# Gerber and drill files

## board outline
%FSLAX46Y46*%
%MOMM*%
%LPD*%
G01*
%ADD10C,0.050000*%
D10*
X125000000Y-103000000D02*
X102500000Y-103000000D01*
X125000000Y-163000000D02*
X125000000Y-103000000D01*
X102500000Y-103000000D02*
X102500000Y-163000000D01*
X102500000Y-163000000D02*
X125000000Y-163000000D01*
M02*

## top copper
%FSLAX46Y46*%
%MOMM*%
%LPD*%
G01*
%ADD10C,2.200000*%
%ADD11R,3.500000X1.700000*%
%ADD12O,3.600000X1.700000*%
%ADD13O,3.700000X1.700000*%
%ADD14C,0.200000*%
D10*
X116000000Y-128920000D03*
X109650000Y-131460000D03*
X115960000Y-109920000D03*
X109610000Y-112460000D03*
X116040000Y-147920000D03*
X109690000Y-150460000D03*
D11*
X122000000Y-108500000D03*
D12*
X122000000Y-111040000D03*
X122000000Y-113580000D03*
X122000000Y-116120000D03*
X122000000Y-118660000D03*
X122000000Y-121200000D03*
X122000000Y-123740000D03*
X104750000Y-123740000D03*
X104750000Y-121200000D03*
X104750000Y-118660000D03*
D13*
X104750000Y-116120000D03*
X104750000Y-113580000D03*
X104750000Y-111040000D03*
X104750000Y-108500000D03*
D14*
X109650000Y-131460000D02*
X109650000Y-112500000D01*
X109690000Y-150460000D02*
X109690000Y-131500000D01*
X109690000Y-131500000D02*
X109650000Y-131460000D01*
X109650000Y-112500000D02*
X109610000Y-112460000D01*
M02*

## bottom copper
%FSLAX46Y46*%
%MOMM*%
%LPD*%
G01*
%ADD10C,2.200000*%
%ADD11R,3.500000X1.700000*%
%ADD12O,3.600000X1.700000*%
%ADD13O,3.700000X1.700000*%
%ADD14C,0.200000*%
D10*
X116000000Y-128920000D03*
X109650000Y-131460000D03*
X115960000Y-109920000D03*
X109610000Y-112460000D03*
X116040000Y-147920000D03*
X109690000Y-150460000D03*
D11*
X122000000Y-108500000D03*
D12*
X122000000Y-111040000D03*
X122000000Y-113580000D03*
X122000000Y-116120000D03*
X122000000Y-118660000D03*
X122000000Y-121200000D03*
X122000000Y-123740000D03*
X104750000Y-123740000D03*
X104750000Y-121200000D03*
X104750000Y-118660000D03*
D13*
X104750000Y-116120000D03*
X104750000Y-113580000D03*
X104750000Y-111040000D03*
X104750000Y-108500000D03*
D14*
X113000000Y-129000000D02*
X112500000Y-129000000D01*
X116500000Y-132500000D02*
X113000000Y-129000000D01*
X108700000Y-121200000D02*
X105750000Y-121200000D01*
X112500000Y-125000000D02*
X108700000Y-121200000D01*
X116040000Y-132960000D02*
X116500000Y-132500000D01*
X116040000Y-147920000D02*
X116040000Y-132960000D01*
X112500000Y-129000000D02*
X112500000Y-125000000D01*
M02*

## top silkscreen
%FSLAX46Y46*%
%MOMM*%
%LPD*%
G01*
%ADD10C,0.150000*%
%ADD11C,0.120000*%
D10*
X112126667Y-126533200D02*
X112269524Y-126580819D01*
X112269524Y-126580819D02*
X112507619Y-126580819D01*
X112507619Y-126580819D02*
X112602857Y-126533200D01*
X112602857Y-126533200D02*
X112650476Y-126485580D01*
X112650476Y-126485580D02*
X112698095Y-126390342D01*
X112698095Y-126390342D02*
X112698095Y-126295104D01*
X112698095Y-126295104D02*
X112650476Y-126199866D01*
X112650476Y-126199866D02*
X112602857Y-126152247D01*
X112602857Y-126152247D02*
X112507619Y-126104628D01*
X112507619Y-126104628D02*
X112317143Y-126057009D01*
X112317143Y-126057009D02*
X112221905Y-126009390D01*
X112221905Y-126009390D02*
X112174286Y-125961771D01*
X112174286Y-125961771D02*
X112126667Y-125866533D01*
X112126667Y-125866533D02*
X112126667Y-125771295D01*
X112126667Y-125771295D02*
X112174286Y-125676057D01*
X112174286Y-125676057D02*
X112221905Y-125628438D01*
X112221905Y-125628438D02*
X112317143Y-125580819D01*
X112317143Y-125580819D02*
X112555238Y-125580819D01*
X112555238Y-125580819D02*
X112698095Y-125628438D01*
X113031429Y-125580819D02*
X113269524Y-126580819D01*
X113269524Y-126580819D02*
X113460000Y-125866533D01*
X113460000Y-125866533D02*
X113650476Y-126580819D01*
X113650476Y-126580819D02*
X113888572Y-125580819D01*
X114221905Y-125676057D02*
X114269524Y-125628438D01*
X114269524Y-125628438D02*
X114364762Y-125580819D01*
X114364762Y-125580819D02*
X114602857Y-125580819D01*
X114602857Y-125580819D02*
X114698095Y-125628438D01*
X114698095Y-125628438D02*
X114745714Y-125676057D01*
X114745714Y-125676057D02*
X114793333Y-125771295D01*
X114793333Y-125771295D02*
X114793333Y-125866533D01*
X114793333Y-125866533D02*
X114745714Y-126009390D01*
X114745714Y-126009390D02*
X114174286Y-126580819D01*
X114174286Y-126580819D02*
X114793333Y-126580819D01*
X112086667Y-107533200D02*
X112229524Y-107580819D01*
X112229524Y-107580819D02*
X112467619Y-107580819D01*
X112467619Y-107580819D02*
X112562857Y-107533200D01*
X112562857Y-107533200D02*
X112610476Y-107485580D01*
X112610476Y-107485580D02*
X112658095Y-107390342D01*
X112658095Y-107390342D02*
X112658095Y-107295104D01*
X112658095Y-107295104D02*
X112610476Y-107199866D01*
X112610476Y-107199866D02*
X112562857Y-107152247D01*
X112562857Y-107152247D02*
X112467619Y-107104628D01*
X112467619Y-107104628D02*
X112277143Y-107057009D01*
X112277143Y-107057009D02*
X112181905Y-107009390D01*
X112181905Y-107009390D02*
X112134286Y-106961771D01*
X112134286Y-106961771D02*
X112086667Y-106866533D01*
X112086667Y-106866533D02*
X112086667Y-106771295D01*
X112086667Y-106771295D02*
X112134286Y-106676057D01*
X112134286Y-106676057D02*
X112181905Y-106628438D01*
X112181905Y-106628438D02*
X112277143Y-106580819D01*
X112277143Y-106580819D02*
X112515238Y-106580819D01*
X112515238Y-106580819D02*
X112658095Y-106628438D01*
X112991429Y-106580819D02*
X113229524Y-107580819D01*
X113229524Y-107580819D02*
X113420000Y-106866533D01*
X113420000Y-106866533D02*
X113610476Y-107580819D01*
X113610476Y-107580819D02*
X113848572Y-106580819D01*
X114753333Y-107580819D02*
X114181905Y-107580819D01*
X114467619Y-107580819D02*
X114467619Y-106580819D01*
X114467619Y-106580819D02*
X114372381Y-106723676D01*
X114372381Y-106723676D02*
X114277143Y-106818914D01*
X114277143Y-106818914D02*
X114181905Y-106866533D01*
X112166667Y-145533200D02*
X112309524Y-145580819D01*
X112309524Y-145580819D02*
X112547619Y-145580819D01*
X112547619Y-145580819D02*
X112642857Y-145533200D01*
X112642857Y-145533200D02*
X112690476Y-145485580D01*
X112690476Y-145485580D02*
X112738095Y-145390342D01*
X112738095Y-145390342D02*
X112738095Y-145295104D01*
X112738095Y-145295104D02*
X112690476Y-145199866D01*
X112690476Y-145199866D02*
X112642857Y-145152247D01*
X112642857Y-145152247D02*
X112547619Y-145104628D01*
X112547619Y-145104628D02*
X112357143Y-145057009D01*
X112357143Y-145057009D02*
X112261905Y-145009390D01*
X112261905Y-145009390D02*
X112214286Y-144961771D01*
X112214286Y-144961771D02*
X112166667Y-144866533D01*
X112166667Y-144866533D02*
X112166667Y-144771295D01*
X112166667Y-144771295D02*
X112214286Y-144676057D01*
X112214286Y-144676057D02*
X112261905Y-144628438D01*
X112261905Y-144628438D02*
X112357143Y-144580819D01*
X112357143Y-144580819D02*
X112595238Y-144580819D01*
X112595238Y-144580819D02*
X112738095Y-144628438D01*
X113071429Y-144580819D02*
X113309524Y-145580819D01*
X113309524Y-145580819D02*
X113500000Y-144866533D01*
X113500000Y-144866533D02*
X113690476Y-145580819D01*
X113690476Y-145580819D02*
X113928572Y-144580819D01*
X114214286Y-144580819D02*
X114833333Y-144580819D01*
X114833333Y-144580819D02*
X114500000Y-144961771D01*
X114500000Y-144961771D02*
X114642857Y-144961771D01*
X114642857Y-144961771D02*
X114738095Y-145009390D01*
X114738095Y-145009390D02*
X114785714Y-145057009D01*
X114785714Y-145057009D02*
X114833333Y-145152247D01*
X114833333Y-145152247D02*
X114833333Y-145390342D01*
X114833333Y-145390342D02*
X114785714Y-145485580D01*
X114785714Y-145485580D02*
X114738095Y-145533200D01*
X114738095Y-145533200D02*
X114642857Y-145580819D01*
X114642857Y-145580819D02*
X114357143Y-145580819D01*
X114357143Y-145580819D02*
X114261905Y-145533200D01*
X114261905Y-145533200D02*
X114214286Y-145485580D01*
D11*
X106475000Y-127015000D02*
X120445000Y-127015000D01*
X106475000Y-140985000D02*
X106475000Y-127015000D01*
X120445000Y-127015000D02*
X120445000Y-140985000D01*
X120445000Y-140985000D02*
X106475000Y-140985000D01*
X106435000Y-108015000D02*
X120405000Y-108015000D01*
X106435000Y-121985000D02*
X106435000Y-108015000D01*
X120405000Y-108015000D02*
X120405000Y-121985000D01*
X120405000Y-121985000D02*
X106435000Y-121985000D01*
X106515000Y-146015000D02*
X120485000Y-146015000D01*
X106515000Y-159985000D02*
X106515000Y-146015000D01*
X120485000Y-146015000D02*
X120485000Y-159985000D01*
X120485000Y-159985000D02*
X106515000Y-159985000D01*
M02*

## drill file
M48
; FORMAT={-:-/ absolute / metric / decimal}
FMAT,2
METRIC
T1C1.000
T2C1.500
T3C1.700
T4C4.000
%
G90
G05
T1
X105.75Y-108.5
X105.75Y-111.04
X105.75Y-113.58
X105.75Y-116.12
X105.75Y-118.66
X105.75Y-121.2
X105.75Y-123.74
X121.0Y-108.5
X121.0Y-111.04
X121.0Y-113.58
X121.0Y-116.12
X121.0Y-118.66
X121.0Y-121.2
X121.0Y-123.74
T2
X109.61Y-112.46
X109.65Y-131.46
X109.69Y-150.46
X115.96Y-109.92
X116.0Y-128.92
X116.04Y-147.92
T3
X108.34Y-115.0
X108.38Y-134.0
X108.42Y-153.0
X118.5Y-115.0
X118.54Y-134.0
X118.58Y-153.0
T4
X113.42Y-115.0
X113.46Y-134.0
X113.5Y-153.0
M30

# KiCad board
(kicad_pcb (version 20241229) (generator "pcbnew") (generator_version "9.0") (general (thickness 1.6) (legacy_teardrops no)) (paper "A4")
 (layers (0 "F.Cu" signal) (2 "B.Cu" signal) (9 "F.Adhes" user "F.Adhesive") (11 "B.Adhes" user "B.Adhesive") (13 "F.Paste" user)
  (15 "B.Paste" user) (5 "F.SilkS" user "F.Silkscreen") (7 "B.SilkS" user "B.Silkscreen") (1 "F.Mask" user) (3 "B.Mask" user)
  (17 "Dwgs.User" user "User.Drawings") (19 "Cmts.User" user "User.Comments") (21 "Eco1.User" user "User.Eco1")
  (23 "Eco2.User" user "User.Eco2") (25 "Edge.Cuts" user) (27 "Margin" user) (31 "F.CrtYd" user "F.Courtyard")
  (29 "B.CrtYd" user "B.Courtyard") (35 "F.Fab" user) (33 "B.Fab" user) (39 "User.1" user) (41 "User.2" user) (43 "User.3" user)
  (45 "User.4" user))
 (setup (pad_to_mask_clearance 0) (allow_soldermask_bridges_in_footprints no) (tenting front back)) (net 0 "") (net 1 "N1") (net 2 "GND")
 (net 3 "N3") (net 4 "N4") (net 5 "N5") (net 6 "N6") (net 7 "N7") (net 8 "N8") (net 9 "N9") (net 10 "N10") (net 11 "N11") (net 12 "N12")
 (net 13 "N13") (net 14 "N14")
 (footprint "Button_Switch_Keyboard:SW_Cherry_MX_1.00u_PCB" (layer "F.Cu") (at 116 128.92)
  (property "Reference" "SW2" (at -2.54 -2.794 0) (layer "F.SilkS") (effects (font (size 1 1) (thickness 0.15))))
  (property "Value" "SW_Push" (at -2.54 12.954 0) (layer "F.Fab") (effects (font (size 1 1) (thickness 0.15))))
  (fp_line (start -9.525 -1.905) (end 4.445 -1.905) (stroke (width 0.12) (type solid)) (layer "F.SilkS"))
  (fp_line (start -9.525 12.065) (end -9.525 -1.905) (stroke (width 0.12) (type solid)) (layer "F.SilkS"))
  (fp_line (start 4.445 -1.905) (end 4.445 12.065) (stroke (width 0.12) (type solid)) (layer "F.SilkS"))
  (fp_line (start 4.445 12.065) (end -9.525 12.065) (stroke (width 0.12) (type solid)) (layer "F.SilkS"))
  (pad "" np_thru_hole circle (at -7.62 5.08) (size 1.7 1.7) (drill 1.7) (layers "*.Cu" "*.Mask"))
  (pad "" np_thru_hole circle (at -2.54 5.08) (size 4 4) (drill 4) (layers "*.Cu" "*.Mask"))
  (pad "" np_thru_hole circle (at 2.54 5.08) (size 1.7 1.7) (drill 1.7) (layers "*.Cu" "*.Mask"))
  (pad "1" thru_hole circle (at 0 0) (size 2.2 2.2) (drill 1.5) (layers "*.Cu" "*.Mask") (remove_unused_layers no) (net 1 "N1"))
  (pad "2" thru_hole circle (at -6.35 2.54) (size 2.2 2.2) (drill 1.5) (layers "*.Cu" "*.Mask") (remove_unused_layers no) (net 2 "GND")))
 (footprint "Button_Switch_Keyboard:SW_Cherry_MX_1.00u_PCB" (layer "F.Cu") (at 115.96 109.92)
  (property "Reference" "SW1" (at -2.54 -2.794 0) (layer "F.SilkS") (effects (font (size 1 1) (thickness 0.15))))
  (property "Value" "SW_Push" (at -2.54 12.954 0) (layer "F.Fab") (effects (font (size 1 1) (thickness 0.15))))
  (fp_line (start -9.525 -1.905) (end 4.445 -1.905) (stroke (width 0.12) (type solid)) (layer "F.SilkS"))
  (fp_line (start -9.525 12.065) (end -9.525 -1.905) (stroke (width 0.12) (type solid)) (layer "F.SilkS"))
  (fp_line (start 4.445 -1.905) (end 4.445 12.065) (stroke (width 0.12) (type solid)) (layer "F.SilkS"))
  (fp_line (start 4.445 12.065) (end -9.525 12.065) (stroke (width 0.12) (type solid)) (layer "F.SilkS"))
  (pad "" np_thru_hole circle (at -7.62 5.08) (size 1.7 1.7) (drill 1.7) (layers "*.Cu" "*.Mask"))
  (pad "" np_thru_hole circle (at -2.54 5.08) (size 4 4) (drill 4) (layers "*.Cu" "*.Mask"))
  (pad "" np_thru_hole circle (at 2.54 5.08) (size 1.7 1.7) (drill 1.7) (layers "*.Cu" "*.Mask"))
  (pad "1" thru_hole circle (at 0 0) (size 2.2 2.2) (drill 1.5) (layers "*.Cu" "*.Mask") (remove_unused_layers no) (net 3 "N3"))
  (pad "2" thru_hole circle (at -6.35 2.54) (size 2.2 2.2) (drill 1.5) (layers "*.Cu" "*.Mask") (remove_unused_layers no) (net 2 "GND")))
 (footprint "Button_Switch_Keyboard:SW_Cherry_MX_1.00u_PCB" (layer "F.Cu") (at 116.04 147.92)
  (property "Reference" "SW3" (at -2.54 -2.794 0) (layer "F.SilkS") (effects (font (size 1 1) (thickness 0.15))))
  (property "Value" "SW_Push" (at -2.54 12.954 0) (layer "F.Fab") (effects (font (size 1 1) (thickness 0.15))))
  (fp_line (start -9.525 -1.905) (end 4.445 -1.905) (stroke (width 0.12) (type solid)) (layer "F.SilkS"))
  (fp_line (start -9.525 12.065) (end -9.525 -1.905) (stroke (width 0.12) (type solid)) (layer "F.SilkS"))
  (fp_line (start 4.445 -1.905) (end 4.445 12.065) (stroke (width 0.12) (type solid)) (layer "F.SilkS"))
  (fp_line (start 4.445 12.065) (end -9.525 12.065) (stroke (width 0.12) (type solid)) (layer "F.SilkS"))
  (pad "" np_thru_hole circle (at -7.62 5.08) (size 1.7 1.7) (drill 1.7) (layers "*.Cu" "*.Mask"))
  (pad "" np_thru_hole circle (at -2.54 5.08) (size 4 4) (drill 4) (layers "*.Cu" "*.Mask"))
  (pad "" np_thru_hole circle (at 2.54 5.08) (size 1.7 1.7) (drill 1.7) (layers "*.Cu" "*.Mask"))
  (pad "1" thru_hole circle (at 0 0) (size 2.2 2.2) (drill 1.5) (layers "*.Cu" "*.Mask") (remove_unused_layers no) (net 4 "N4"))
  (pad "2" thru_hole circle (at -6.35 2.54) (size 2.2 2.2) (drill 1.5) (layers "*.Cu" "*.Mask") (remove_unused_layers no) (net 2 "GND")))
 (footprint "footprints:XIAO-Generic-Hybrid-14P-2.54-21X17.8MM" (layer "B.Cu") (at 113.375 116.12 180)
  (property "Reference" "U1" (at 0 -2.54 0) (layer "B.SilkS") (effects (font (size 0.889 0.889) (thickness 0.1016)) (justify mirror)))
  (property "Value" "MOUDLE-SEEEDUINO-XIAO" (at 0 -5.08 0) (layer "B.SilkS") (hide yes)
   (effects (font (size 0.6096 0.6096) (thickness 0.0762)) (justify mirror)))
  (pad "1" thru_hole rect (at -7.625 7.62 180) (size 3.5 1.7) (drill 1 (offset -1 0)) (layers "*.Cu" "*.Mask") (remove_unused_layers no)
   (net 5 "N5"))
  (pad "2" thru_hole oval (at -7.625 5.08 180) (size 3.6 1.7) (drill 1 (offset -1 0)) (layers "*.Cu" "*.Mask") (remove_unused_layers no)
   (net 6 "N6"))
  (pad "3" thru_hole oval (at -7.625 2.54 180) (size 3.6 1.7) (drill 1 (offset -1 0)) (layers "*.Cu" "*.Mask") (remove_unused_layers no)
   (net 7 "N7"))
  (pad "4" thru_hole oval (at -7.625 0 180) (size 3.6 1.7) (drill 1 (offset -1 0)) (layers "*.Cu" "*.Mask") (remove_unused_layers no)
   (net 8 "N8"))
  (pad "5" thru_hole oval (at -7.625 -2.54 180) (size 3.6 1.7) (drill 1 (offset -1 0)) (layers "*.Cu" "*.Mask") (remove_unused_layers no)
   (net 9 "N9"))
  (pad "6" thru_hole oval (at -7.625 -5.08) (size 3.6 1.7) (drill 1 (offset 1 0)) (layers "*.Cu" "*.Mask") (remove_unused_layers no)
   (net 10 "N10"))
  (pad "7" thru_hole oval (at -7.625 -7.62 180) (size 3.6 1.7) (drill 1 (offset -1 0)) (layers "*.Cu" "*.Mask") (remove_unused_layers no)
   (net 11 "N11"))
  (pad "8" thru_hole oval (at 7.625 -7.62 180) (size 3.6 1.7) (drill 1 (offset 1 0)) (layers "*.Cu" "*.Mask") (remove_unused_layers no)
   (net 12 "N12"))
  (pad "9" thru_hole oval (at 7.625 -5.08 180) (size 3.6 1.7) (drill 1 (offset 1 0)) (layers "*.Cu" "*.Mask") (remove_unused_layers no)
   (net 4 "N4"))
  (pad "10" thru_hole oval (at 7.625 -2.54 180) (size 3.6 1.7) (drill 1 (offset 1 0)) (layers "*.Cu" "*.Mask") (remove_unused_layers no)
   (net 1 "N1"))
  (pad "11" thru_hole oval (at 7.625 0 180) (size 3.7 1.7) (drill 1 (offset 1 0)) (layers "*.Cu" "*.Mask") (remove_unused_layers no)
   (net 3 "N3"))
  (pad "12" thru_hole oval (at 7.625 2.54 180) (size 3.7 1.7) (drill 1 (offset 1 0)) (layers "*.Cu" "*.Mask") (remove_unused_layers no)
   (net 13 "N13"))
  (pad "13" thru_hole oval (at 7.625 5.08 180) (size 3.7 1.7) (drill 1 (offset 1 0)) (layers "*.Cu" "*.Mask") (remove_unused_layers no)
   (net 2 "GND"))
  (pad "14" thru_hole oval (at 7.625 7.62 180) (size 3.7 1.7) (drill 1 (offset 1 0)) (layers "*.Cu" "*.Mask") (remove_unused_layers no)
   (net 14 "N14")))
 (gr_line (start 125 103) (end 102.5 103) (stroke (width 0.05) (type default)) (layer "Edge.Cuts"))
 (gr_line (start 125 163) (end 125 103) (stroke (width 0.05) (type default)) (layer "Edge.Cuts"))
 (gr_line (start 102.5 103) (end 102.5 163) (stroke (width 0.05) (type default)) (layer "Edge.Cuts"))
 (gr_line (start 102.5 163) (end 125 163) (stroke (width 0.05) (type default)) (layer "Edge.Cuts"))
 (segment (start 109.65 131.46) (end 109.65 112.5) (width 0.2) (layer "F.Cu") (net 2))
 (segment (start 109.69 150.46) (end 109.69 131.5) (width 0.2) (layer "F.Cu") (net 2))
 (segment (start 109.69 131.5) (end 109.65 131.46) (width 0.2) (layer "F.Cu") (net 2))
 (segment (start 109.65 112.5) (end 109.61 112.46) (width 0.2) (layer "F.Cu") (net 2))
 (segment (start 113 129) (end 112.5 129) (width 0.2) (layer "B.Cu") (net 4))
 (segment (start 116.5 132.5) (end 113 129) (width 0.2) (layer "B.Cu") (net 4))
 (segment (start 108.7 121.2) (end 105.75 121.2) (width 0.2) (layer "B.Cu") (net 4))
 (segment (start 112.5 125) (end 108.7 121.2) (width 0.2) (layer "B.Cu") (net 4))
 (segment (start 116.04 132.96) (end 116.5 132.5) (width 0.2) (layer "B.Cu") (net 4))
 (segment (start 116.04 147.92) (end 116.04 132.96) (width 0.2) (layer "B.Cu") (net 4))
 (segment (start 112.5 129) (end 112.5 125) (width 0.2) (layer "B.Cu") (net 4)))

